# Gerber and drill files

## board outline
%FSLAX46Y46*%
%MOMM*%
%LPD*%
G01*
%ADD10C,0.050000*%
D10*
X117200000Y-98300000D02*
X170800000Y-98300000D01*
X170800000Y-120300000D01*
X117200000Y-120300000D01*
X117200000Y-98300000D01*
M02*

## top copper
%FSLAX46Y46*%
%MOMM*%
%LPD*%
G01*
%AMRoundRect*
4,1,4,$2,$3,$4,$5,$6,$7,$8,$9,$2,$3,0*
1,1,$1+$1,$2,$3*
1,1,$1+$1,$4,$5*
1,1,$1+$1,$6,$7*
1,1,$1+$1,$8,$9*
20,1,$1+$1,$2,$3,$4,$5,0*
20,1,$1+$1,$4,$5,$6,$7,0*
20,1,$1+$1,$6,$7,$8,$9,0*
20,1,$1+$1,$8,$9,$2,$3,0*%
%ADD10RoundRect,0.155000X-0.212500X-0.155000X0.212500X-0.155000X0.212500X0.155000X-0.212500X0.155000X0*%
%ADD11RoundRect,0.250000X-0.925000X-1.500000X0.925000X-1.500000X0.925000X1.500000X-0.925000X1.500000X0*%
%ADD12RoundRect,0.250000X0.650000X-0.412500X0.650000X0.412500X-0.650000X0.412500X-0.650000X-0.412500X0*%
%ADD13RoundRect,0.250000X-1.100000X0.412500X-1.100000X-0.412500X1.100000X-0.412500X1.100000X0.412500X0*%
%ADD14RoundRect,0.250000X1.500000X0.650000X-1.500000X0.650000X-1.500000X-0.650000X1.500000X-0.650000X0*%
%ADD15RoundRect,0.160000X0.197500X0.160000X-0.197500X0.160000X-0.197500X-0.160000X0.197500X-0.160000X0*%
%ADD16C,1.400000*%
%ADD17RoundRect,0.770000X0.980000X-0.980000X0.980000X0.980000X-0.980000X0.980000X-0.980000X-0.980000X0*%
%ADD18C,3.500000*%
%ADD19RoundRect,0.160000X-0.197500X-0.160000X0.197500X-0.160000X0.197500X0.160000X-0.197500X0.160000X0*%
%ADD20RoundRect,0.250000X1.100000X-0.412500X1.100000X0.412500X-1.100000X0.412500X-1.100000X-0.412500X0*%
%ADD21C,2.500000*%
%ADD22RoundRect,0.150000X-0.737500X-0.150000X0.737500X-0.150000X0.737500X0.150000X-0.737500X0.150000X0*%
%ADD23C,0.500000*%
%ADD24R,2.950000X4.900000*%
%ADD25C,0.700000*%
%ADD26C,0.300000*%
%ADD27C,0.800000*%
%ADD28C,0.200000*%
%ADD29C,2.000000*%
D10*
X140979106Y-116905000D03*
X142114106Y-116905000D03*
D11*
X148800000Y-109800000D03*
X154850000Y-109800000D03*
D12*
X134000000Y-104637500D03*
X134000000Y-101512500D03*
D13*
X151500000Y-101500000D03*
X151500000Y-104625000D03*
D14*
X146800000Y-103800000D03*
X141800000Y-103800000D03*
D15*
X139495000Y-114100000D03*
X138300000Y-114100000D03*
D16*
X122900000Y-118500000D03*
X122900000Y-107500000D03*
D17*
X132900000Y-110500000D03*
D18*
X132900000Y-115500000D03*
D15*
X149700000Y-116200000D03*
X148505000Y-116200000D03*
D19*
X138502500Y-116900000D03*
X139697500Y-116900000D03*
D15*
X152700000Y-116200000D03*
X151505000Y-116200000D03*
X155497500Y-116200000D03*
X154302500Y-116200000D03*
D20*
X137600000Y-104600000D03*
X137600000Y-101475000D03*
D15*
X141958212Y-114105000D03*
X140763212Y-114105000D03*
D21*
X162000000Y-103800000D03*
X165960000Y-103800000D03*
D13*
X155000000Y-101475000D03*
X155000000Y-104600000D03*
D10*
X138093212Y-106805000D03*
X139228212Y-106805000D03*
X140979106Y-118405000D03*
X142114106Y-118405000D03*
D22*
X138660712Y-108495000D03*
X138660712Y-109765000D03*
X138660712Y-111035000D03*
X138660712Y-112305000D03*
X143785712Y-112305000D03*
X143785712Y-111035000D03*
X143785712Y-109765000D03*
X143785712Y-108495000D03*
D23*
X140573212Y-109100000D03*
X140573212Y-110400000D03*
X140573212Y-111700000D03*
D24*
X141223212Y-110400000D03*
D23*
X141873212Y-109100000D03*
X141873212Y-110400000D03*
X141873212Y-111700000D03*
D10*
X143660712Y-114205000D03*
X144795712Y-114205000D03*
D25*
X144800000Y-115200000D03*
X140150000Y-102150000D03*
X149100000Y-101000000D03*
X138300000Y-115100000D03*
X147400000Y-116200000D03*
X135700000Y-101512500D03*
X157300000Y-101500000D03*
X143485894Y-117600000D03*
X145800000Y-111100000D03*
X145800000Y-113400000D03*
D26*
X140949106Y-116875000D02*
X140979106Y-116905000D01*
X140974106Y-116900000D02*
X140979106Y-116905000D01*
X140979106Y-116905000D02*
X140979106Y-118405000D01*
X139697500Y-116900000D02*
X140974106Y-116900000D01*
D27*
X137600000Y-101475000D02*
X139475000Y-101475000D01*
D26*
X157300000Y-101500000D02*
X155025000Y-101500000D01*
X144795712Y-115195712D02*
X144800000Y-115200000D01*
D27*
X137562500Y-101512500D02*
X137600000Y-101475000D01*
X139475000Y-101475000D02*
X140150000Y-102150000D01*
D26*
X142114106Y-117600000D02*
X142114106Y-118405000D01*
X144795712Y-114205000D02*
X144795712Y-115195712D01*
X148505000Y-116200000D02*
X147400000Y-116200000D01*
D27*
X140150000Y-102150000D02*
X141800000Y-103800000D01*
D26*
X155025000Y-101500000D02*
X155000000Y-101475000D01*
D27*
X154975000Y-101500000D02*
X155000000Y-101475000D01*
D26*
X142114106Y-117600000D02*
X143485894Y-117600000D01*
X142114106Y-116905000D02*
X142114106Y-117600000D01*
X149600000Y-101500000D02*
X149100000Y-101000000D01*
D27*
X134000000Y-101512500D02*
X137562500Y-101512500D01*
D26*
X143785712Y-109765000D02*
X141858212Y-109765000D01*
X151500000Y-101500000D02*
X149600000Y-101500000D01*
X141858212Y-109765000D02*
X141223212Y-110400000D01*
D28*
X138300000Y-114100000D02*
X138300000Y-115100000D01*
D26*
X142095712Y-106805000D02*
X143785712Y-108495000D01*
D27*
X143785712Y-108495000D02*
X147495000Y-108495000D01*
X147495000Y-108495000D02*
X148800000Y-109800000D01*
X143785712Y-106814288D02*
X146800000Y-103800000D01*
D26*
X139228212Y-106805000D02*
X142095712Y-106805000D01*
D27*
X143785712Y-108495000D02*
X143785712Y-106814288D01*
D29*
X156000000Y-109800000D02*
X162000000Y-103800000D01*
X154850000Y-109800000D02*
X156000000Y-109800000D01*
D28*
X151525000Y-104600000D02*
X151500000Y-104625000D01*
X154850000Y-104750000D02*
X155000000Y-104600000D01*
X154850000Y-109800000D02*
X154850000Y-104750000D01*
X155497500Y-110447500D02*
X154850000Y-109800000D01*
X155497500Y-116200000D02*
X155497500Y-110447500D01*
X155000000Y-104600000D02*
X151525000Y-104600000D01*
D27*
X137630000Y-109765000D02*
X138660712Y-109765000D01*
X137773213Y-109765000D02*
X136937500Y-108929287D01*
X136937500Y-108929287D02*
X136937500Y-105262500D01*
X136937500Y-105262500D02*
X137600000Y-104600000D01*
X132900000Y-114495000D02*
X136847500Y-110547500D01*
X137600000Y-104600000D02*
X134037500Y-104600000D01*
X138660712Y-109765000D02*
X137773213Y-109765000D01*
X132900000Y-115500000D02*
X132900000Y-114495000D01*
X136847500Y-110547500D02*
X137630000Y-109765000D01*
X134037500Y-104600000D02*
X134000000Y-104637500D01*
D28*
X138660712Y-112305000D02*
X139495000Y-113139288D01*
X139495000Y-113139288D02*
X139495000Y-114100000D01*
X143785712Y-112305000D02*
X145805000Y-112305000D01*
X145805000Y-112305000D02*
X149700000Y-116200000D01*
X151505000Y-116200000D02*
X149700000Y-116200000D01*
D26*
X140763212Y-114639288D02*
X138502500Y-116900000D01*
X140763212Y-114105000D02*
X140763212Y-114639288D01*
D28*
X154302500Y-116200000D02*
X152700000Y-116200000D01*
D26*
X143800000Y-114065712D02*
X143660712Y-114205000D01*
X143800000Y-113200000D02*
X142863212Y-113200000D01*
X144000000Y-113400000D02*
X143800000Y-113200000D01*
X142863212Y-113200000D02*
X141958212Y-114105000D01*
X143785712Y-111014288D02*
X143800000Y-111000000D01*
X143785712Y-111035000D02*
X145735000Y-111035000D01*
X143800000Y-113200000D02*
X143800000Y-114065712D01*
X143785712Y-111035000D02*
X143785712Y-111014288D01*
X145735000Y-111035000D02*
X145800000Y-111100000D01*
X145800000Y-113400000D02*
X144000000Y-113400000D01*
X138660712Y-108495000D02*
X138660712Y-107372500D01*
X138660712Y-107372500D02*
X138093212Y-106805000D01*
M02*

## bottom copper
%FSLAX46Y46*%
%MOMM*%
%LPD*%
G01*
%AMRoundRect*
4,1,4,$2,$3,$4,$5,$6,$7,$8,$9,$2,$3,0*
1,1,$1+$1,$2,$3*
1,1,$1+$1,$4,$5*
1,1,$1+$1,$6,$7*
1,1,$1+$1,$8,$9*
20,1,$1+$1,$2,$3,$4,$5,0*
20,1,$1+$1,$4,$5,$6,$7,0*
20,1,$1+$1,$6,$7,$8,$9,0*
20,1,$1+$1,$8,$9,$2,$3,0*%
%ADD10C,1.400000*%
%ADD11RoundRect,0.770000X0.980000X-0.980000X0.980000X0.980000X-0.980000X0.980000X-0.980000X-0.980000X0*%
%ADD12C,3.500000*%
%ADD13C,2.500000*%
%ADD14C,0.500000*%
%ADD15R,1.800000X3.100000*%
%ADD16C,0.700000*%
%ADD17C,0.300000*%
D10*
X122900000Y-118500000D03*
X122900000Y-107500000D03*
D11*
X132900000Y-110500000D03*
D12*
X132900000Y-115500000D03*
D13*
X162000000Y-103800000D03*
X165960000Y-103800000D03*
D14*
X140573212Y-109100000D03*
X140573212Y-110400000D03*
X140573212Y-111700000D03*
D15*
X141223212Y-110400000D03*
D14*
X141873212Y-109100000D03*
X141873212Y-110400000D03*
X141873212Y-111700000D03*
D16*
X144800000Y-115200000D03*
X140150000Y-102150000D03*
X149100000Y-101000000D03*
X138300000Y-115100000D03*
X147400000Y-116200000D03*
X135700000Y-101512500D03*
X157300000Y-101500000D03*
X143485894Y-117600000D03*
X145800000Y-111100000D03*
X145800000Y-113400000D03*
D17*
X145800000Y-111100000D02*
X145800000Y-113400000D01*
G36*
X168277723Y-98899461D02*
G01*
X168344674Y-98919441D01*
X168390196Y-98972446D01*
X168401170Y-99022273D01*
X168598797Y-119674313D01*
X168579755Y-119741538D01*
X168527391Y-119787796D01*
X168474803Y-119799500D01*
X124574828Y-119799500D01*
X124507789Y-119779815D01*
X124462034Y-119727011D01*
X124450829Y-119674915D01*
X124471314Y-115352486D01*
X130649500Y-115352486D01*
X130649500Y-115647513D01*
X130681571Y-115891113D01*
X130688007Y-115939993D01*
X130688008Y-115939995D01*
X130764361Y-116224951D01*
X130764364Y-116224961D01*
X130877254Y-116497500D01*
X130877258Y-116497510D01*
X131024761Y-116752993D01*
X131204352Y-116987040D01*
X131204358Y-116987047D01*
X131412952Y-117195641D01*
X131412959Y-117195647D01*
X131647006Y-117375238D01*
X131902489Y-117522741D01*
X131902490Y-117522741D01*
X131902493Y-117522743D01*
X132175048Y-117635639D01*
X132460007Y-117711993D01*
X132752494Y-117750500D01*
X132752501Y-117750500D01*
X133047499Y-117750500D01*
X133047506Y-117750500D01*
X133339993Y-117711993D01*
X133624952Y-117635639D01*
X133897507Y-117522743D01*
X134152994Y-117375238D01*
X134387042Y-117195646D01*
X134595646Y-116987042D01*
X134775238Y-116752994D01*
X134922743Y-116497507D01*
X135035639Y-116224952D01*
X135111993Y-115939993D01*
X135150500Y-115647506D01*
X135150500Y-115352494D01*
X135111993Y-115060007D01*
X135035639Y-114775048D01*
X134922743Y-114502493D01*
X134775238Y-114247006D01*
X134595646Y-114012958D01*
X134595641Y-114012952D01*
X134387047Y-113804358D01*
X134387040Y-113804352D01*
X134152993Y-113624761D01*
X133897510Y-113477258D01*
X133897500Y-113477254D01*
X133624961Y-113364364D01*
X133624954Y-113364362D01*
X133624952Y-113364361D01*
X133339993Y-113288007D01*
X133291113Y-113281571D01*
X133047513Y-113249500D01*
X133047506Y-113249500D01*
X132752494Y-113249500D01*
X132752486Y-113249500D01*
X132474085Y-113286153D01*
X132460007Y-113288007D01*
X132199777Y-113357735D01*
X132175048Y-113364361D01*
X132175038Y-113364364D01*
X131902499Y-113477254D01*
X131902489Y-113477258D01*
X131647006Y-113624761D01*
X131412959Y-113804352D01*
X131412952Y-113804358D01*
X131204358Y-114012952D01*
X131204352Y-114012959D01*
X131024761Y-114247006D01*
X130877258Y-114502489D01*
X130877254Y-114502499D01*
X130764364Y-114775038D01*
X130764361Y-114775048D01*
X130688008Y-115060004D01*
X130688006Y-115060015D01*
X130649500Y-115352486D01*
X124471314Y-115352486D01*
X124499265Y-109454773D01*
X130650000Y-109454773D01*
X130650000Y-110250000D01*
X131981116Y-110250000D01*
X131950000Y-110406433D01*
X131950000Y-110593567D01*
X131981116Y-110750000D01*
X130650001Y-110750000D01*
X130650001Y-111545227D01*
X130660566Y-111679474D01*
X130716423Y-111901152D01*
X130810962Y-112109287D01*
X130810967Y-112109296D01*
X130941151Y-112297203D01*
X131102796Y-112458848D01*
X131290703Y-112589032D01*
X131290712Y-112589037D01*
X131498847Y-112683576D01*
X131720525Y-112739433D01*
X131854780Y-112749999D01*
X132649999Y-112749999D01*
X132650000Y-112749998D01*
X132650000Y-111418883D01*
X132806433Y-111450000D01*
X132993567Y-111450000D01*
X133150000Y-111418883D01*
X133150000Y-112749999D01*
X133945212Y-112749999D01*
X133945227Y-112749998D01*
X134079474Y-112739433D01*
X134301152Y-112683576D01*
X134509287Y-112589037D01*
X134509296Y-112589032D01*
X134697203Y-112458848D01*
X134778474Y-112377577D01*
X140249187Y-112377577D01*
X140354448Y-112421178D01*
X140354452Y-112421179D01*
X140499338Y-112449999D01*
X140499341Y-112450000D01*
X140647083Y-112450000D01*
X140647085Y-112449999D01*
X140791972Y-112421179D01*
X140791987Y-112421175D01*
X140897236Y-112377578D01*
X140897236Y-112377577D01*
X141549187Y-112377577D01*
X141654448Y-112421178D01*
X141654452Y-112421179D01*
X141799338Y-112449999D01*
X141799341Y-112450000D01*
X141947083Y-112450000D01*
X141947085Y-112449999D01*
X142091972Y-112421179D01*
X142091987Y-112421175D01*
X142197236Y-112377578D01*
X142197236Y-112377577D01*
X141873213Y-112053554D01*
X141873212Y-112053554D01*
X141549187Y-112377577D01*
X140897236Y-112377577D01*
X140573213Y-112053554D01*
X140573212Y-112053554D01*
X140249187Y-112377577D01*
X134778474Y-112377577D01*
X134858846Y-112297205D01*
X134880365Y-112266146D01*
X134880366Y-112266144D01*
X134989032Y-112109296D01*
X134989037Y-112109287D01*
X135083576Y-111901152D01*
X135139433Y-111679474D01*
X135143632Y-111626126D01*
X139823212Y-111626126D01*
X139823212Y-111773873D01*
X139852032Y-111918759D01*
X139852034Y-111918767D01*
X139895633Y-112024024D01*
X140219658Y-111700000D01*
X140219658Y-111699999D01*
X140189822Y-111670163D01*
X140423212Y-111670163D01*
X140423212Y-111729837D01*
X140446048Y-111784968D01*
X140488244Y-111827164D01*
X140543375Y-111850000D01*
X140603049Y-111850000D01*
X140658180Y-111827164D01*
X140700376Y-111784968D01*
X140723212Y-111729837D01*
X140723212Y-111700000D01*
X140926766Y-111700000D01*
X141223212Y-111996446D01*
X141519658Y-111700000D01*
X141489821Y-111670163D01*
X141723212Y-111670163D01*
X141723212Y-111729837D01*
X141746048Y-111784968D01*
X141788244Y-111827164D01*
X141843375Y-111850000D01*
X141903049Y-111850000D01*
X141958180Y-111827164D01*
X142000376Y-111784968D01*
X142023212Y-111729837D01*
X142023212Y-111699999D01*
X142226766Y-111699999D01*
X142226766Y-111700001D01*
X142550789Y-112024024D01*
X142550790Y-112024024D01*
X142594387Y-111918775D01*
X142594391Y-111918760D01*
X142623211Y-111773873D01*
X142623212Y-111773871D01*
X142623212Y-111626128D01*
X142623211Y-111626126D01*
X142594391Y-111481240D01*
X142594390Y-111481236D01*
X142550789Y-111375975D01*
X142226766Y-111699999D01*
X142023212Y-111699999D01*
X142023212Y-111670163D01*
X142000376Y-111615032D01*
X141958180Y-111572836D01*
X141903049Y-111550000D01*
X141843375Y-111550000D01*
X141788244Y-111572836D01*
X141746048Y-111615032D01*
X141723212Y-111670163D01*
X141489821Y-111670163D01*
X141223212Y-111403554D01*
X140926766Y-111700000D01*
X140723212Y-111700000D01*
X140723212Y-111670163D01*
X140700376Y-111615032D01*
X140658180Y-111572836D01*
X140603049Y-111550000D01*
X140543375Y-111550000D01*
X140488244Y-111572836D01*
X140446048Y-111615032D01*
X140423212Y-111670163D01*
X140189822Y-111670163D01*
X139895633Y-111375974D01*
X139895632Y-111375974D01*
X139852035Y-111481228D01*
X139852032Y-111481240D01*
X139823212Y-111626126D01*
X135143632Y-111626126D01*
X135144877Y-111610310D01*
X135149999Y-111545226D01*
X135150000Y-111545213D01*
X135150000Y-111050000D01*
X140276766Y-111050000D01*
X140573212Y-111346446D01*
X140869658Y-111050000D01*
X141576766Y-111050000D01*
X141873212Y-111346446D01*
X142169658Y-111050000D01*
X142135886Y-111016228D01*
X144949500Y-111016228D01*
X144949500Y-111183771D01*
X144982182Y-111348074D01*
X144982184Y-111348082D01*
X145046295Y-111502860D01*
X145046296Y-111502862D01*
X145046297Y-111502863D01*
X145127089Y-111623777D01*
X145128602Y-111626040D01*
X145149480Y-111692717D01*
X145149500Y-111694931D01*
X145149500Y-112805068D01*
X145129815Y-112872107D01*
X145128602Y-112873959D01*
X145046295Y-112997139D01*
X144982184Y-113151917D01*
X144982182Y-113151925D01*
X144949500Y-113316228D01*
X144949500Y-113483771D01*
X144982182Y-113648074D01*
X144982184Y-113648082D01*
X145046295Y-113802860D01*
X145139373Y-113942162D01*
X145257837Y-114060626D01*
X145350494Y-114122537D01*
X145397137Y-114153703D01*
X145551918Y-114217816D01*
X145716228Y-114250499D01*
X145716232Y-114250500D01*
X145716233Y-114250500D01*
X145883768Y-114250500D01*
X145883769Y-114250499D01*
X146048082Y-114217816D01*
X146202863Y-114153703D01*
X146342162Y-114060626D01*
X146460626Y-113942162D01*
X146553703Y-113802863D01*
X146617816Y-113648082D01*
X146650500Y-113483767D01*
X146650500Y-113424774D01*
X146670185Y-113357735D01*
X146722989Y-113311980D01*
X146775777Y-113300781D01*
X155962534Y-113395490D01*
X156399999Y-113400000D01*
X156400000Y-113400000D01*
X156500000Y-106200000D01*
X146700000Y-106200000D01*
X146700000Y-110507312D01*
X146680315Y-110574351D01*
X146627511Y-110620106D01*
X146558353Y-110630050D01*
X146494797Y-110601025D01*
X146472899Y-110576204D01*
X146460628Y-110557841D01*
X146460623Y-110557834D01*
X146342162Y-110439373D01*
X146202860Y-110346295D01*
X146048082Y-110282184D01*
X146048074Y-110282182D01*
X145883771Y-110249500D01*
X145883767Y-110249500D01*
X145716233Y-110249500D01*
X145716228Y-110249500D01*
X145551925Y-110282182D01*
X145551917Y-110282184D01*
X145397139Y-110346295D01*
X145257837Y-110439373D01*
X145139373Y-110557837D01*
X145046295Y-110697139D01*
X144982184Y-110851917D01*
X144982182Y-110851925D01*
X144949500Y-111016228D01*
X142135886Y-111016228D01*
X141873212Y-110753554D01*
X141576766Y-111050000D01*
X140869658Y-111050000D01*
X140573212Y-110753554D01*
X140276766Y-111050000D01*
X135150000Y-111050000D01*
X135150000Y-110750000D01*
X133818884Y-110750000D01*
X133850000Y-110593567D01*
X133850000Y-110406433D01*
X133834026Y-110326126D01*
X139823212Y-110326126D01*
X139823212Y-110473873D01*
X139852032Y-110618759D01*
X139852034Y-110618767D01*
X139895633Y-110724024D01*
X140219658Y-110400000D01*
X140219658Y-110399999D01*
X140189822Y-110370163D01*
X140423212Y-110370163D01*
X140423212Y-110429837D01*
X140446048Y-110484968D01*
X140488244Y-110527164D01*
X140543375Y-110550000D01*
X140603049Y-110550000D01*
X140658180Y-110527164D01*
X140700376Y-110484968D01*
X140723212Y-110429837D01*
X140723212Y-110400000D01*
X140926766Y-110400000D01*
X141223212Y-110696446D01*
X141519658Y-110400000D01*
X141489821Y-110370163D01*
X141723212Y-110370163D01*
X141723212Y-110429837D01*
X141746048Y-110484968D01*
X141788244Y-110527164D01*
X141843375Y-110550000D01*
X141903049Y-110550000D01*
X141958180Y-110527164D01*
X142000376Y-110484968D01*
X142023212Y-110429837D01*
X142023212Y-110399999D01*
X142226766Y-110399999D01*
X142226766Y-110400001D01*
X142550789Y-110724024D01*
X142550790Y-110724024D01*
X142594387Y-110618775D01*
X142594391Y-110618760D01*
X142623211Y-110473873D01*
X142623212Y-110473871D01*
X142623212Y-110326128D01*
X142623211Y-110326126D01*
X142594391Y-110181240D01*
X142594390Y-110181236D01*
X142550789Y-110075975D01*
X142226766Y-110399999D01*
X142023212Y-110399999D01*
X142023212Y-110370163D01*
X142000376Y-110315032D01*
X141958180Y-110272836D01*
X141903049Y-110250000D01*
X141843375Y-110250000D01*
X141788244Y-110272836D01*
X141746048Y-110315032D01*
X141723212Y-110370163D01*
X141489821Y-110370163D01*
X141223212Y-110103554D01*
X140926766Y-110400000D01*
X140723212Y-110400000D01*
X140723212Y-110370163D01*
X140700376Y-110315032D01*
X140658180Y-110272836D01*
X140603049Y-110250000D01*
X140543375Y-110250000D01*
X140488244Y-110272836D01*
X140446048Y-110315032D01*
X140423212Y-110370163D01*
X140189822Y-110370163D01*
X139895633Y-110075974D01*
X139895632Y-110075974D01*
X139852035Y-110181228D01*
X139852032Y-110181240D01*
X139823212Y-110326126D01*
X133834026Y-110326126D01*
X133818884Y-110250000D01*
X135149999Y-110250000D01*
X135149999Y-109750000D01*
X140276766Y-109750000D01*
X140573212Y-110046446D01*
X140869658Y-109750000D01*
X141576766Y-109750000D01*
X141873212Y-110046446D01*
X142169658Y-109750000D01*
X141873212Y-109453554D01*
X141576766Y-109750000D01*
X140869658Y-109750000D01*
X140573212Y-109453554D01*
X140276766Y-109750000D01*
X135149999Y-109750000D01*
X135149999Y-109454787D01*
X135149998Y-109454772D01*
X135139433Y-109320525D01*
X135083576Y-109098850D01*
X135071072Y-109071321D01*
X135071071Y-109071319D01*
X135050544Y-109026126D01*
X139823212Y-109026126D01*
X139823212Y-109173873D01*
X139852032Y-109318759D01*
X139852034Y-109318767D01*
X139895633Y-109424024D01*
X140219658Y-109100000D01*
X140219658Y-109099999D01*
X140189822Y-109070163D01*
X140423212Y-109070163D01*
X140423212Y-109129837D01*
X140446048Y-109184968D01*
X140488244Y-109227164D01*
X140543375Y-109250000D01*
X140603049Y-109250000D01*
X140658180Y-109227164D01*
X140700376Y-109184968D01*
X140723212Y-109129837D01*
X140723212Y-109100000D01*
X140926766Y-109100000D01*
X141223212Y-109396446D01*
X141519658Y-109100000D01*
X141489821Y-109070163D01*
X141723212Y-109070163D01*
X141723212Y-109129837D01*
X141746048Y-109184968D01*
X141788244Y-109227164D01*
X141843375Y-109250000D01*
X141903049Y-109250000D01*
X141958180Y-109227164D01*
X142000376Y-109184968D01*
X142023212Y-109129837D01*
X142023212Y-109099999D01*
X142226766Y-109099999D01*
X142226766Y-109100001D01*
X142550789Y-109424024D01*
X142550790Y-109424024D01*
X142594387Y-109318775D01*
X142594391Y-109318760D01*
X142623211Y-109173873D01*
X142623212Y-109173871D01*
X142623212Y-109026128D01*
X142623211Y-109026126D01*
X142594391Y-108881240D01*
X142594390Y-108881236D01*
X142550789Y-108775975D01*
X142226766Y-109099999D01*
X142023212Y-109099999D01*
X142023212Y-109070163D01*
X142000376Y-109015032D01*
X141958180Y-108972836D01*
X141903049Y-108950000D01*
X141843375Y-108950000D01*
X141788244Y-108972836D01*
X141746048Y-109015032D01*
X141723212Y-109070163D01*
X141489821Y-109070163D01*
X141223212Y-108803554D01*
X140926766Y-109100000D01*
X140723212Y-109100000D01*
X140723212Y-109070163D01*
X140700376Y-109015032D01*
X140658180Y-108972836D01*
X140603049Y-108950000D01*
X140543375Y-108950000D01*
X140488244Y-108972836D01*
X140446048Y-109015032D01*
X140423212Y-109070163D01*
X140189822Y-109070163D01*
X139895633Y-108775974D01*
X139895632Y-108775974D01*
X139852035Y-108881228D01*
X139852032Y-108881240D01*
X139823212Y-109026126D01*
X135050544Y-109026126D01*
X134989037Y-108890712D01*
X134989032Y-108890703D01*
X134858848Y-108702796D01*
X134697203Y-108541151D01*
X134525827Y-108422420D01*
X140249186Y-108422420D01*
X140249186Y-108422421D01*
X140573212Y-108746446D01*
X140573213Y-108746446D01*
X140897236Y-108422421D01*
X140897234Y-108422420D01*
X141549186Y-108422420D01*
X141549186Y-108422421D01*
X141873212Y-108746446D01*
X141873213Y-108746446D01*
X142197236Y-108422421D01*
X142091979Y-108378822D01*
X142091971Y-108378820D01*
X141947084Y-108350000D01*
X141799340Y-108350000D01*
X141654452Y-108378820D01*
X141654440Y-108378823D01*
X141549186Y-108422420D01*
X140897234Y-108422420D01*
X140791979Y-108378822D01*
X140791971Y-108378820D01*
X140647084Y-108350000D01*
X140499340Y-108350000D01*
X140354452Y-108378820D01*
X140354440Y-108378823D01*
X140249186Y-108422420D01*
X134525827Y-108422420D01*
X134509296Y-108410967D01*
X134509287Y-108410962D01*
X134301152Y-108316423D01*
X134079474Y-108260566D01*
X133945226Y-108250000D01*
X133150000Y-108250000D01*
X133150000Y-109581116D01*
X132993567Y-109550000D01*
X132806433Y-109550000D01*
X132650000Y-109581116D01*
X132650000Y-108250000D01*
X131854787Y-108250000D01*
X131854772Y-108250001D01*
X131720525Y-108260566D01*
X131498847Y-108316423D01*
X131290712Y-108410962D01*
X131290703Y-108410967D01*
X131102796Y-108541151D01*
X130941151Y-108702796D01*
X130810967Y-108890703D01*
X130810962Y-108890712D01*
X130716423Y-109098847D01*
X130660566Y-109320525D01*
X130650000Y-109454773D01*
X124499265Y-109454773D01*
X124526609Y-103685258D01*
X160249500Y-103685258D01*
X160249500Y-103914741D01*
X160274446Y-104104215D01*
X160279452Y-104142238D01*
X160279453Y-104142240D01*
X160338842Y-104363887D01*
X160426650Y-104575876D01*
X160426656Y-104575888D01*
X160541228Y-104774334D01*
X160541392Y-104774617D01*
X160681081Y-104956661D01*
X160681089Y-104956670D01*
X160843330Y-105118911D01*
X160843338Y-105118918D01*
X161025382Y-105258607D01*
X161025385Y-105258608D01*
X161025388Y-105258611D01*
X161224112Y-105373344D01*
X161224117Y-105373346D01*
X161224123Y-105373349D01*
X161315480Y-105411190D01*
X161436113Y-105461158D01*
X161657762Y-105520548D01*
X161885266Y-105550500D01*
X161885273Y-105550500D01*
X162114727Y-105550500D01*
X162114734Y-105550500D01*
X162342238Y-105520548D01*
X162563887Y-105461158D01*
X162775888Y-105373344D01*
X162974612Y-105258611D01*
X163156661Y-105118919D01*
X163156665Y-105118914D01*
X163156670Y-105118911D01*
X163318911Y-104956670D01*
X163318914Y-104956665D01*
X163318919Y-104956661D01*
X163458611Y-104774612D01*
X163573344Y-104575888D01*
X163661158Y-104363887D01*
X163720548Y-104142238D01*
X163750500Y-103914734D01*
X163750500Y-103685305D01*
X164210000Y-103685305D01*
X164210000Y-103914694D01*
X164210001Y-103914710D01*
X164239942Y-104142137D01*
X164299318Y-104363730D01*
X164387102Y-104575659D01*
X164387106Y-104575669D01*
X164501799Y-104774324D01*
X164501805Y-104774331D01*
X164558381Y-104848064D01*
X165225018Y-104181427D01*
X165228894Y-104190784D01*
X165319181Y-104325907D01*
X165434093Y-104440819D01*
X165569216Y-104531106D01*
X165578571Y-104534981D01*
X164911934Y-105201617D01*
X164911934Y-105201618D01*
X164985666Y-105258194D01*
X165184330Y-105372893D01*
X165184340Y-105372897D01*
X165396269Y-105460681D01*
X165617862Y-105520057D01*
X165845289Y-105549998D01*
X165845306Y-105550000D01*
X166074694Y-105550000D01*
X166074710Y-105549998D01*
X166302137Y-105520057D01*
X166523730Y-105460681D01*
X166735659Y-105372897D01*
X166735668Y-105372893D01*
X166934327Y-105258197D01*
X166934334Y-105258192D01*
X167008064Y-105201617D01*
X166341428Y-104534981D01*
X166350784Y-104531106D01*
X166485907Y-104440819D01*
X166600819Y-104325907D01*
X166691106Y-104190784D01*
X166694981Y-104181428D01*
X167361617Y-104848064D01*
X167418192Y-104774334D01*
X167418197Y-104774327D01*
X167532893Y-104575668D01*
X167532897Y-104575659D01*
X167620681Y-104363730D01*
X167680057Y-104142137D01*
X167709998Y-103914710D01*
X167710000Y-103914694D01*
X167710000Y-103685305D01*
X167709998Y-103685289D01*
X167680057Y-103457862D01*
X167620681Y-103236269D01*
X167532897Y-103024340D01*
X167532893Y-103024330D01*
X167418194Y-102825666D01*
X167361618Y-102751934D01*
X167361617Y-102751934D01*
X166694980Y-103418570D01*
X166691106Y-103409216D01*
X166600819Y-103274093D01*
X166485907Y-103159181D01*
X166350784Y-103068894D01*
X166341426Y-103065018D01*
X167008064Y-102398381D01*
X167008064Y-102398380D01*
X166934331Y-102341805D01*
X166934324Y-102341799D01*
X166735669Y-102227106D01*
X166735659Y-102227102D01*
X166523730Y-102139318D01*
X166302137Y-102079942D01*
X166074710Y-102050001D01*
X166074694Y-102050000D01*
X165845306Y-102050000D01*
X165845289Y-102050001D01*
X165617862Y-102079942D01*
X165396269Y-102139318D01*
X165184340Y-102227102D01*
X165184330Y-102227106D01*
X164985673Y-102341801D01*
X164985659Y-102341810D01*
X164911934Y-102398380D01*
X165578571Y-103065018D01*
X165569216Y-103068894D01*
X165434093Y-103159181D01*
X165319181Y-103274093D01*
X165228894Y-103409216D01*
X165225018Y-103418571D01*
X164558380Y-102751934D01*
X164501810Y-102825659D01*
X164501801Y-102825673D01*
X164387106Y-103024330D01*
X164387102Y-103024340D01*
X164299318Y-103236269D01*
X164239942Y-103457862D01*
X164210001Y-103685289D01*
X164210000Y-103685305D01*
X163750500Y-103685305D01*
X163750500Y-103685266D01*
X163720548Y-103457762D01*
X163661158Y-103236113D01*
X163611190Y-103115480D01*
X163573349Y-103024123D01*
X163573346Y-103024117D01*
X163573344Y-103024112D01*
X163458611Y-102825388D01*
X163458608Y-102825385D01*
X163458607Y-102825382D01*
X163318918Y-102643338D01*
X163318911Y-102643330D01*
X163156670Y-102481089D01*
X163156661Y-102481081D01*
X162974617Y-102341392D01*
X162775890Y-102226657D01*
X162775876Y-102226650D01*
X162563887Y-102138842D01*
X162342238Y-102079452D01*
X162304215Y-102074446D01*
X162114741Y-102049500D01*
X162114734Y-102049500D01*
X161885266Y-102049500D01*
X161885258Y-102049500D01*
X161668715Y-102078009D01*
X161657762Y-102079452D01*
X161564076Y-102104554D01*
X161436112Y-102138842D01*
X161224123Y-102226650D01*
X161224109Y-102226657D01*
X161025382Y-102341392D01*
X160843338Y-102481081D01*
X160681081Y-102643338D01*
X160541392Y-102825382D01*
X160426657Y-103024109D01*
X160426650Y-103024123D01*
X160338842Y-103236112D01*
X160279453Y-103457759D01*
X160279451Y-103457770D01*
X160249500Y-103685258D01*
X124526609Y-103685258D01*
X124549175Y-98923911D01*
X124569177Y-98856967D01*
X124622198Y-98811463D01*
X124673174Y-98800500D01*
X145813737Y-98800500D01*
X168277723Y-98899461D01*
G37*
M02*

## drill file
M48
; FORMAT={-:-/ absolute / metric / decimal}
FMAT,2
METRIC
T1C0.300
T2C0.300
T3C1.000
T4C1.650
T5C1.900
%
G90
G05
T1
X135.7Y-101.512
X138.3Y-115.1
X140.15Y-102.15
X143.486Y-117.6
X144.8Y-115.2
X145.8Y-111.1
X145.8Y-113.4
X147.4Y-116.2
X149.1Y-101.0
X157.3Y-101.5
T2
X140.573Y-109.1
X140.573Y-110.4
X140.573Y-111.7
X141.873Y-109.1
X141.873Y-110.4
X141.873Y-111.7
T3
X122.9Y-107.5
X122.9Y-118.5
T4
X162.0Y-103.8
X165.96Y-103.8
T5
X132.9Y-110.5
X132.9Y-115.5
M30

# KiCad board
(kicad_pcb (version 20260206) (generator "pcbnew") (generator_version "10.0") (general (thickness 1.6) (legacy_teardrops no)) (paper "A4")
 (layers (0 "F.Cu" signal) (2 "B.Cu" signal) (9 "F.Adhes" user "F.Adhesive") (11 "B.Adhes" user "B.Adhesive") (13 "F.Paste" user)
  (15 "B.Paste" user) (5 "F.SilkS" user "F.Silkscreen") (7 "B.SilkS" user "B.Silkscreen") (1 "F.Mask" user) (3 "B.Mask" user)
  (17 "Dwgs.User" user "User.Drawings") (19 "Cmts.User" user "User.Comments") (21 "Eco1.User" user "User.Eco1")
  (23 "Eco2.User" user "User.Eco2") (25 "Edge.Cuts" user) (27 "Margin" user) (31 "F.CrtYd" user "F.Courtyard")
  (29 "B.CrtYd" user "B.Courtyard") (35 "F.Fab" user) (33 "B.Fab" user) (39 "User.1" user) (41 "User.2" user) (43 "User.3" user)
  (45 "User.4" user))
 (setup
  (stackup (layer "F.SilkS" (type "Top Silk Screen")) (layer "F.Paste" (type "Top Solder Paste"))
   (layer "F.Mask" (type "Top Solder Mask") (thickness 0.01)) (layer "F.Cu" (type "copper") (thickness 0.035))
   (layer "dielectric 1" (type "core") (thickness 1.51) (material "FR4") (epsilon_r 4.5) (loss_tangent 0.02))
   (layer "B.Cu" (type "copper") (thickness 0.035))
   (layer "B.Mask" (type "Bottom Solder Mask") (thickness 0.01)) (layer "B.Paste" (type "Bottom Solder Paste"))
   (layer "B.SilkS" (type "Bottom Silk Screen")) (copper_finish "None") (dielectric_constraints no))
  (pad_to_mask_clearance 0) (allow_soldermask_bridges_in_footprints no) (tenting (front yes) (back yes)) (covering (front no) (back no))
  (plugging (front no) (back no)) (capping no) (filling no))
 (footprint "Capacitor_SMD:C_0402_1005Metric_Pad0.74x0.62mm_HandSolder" (layer "F.Cu") (at 141.546606 116.905)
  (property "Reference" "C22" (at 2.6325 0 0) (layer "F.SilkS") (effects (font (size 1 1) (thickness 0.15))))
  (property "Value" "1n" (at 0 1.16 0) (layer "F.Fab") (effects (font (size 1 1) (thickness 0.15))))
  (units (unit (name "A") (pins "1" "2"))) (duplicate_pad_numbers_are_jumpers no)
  (pad "1" smd roundrect (at -0.5675 0) (size 0.735 0.62) (layers "F.Cu" "F.Mask" "F.Paste") (roundrect_rratio 0.25) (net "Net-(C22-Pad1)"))
  (pad "2" smd roundrect (at 0.5675 0) (size 0.735 0.62) (layers "F.Cu" "F.Mask" "F.Paste") (roundrect_rratio 0.25) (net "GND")))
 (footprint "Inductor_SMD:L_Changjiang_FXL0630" (layer "F.Cu") (at 151.825 109.8)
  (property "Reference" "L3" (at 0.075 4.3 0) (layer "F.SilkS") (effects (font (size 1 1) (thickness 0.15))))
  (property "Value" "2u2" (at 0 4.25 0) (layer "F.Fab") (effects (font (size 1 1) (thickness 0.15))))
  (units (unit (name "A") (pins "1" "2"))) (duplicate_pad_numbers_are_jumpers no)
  (pad "1" smd roundrect (at -3.025 0) (size 2.35 3.5) (layers "F.Cu" "F.Mask" "F.Paste") (roundrect_rratio 0.106383) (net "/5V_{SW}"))
  (pad "2" smd roundrect (at 3.025 0) (size 2.35 3.5) (layers "F.Cu" "F.Mask" "F.Paste") (roundrect_rratio 0.106383) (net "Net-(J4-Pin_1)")))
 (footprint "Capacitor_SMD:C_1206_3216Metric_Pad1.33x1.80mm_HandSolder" (layer "F.Cu") (at 134 103.075 90)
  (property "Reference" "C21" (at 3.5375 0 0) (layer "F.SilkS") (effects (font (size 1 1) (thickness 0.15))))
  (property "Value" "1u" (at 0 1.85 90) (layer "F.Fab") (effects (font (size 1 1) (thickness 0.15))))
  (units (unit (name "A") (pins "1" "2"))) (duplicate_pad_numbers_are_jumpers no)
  (pad "1" smd roundrect (at -1.5625 0 90) (size 1.325 1.8) (layers "F.Cu" "F.Mask" "F.Paste") (roundrect_rratio 0.188679) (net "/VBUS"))
  (pad "2" smd roundrect (at 1.5625 0 90) (size 1.325 1.8) (layers "F.Cu" "F.Mask" "F.Paste") (roundrect_rratio 0.188679) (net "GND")))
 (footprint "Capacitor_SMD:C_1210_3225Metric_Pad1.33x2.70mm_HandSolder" (layer "F.Cu") (at 151.5 103.0625 -90)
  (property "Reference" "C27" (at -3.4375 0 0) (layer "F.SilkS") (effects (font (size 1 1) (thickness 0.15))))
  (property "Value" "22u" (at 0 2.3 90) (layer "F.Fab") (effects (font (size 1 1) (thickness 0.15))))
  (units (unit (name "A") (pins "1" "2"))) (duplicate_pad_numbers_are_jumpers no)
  (pad "1" smd roundrect (at -1.5625 0 270) (size 1.325 2.7) (layers "F.Cu" "F.Mask" "F.Paste") (roundrect_rratio 0.188679) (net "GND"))
  (pad "2" smd roundrect (at 1.5625 0 270) (size 1.325 2.7) (layers "F.Cu" "F.Mask" "F.Paste") (roundrect_rratio 0.188679)
   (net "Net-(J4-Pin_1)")))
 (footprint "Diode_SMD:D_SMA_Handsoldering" (layer "F.Cu") (at 144.3 103.8 180)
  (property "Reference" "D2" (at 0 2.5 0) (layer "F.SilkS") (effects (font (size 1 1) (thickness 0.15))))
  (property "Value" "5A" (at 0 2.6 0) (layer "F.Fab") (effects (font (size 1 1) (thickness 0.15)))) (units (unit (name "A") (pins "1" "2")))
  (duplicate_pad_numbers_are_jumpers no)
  (pad "1" smd roundrect (at -2.5 0 180) (size 3.5 1.8) (layers "F.Cu" "F.Mask" "F.Paste") (roundrect_rratio 0.1388888889) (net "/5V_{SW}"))
  (pad "2" smd roundrect (at 2.5 0 180) (size 3.5 1.8) (layers "F.Cu" "F.Mask" "F.Paste") (roundrect_rratio 0.1388888889) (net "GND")))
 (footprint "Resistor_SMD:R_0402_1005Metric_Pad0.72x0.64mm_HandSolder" (layer "F.Cu") (at 138.8975 114.1 180)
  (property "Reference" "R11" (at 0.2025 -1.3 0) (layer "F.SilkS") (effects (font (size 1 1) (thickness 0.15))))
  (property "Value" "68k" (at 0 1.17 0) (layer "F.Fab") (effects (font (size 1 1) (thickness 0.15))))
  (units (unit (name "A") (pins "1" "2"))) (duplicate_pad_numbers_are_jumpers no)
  (pad "1" smd roundrect (at -0.5975 0 180) (size 0.715 0.64) (layers "F.Cu" "F.Mask" "F.Paste") (roundrect_rratio 0.25) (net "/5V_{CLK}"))
  (pad "2" smd roundrect (at 0.5975 0 180) (size 0.715 0.64) (layers "F.Cu" "F.Mask" "F.Paste") (roundrect_rratio 0.25) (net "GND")))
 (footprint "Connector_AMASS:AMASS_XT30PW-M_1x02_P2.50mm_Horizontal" (layer "F.Cu") (at 132.9 110.5 90)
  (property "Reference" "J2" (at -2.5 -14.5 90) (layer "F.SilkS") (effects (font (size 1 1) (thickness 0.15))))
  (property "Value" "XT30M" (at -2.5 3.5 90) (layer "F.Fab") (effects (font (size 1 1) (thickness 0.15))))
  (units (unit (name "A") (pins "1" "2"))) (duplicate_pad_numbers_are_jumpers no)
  (pad "" thru_hole circle (at -8 -10 90) (size 1.4 1.4) (drill 1) (layers "*.Cu" "*.Mask") (remove_unused_layers no))
  (pad "" thru_hole circle (at 3 -10 90) (size 1.4 1.4) (drill 1) (layers "*.Cu" "*.Mask") (remove_unused_layers no))
  (pad "1" thru_hole roundrect (at 0 0 90) (size 3.5 3.5) (drill 1.9) (layers "*.Cu" "*.Mask") (remove_unused_layers no)
   (roundrect_rratio 0.22) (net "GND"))
  (pad "2" thru_hole circle (at -5 0 90) (size 3.5 3.5) (drill 1.9) (layers "*.Cu" "*.Mask") (remove_unused_layers no) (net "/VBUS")))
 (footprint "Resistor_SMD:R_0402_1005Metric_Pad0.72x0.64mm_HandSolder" (layer "F.Cu") (at 149.1025 116.2 180)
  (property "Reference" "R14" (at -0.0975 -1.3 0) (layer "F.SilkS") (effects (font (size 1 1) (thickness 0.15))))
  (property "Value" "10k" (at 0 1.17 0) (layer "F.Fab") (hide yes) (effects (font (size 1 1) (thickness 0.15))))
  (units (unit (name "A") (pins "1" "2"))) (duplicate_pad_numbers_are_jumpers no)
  (pad "1" smd roundrect (at -0.5975 0 180) (size 0.715 0.64) (layers "F.Cu" "F.Mask" "F.Paste") (roundrect_rratio 0.25) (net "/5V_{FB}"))
  (pad "2" smd roundrect (at 0.5975 0 180) (size 0.715 0.64) (layers "F.Cu" "F.Mask" "F.Paste") (roundrect_rratio 0.25) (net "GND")))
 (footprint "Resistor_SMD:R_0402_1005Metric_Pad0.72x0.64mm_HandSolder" (layer "F.Cu") (at 139.1 116.9)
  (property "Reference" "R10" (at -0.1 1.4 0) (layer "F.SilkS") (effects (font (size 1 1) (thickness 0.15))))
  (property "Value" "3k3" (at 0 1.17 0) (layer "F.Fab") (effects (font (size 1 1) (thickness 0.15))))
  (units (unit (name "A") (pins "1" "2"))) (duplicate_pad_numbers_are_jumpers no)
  (pad "1" smd roundrect (at -0.5975 0) (size 0.715 0.64) (layers "F.Cu" "F.Mask" "F.Paste") (roundrect_rratio 0.25) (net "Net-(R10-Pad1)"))
  (pad "2" smd roundrect (at 0.5975 0) (size 0.715 0.64) (layers "F.Cu" "F.Mask" "F.Paste") (roundrect_rratio 0.25) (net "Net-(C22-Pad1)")))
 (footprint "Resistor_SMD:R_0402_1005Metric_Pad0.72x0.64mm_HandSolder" (layer "F.Cu") (at 152.1025 116.2 180)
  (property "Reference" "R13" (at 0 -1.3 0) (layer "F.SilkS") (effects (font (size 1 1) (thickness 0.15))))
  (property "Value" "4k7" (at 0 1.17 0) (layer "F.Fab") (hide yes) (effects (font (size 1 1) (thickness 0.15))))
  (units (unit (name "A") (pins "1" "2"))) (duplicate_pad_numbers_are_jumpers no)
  (pad "1" smd roundrect (at -0.5975 0 180) (size 0.715 0.64) (layers "F.Cu" "F.Mask" "F.Paste") (roundrect_rratio 0.25)
   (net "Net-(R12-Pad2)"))
  (pad "2" smd roundrect (at 0.5975 0 180) (size 0.715 0.64) (layers "F.Cu" "F.Mask" "F.Paste") (roundrect_rratio 0.25) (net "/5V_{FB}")))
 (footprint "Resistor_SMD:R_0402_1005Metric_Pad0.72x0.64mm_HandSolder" (layer "F.Cu") (at 154.9 116.2 180)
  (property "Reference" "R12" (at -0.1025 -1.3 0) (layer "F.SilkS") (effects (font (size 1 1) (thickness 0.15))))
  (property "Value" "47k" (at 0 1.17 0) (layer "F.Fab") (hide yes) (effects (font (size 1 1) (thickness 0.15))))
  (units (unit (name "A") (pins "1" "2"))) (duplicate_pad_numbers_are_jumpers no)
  (pad "1" smd roundrect (at -0.5975 0 180) (size 0.715 0.64) (layers "F.Cu" "F.Mask" "F.Paste") (roundrect_rratio 0.25)
   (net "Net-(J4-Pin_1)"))
  (pad "2" smd roundrect (at 0.5975 0 180) (size 0.715 0.64) (layers "F.Cu" "F.Mask" "F.Paste") (roundrect_rratio 0.25)
   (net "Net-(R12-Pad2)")))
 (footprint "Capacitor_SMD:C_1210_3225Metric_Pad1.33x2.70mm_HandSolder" (layer "F.Cu") (at 137.6 103.0375 90)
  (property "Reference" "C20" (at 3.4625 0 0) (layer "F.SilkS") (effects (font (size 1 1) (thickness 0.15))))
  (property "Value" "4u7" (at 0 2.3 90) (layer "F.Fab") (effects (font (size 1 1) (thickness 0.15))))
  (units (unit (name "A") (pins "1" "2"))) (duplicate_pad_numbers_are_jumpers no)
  (pad "1" smd roundrect (at -1.5625 0 90) (size 1.325 2.7) (layers "F.Cu" "F.Mask" "F.Paste") (roundrect_rratio 0.188679) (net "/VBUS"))
  (pad "2" smd roundrect (at 1.5625 0 90) (size 1.325 2.7) (layers "F.Cu" "F.Mask" "F.Paste") (roundrect_rratio 0.188679) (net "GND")))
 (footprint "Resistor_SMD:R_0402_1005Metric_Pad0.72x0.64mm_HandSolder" (layer "F.Cu") (at 141.360712 114.105 180)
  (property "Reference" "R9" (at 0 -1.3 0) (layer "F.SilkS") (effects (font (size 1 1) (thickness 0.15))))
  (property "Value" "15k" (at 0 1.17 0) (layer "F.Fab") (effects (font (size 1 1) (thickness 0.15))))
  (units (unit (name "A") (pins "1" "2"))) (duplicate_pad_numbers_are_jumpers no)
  (pad "1" smd roundrect (at -0.5975 0 180) (size 0.715 0.64) (layers "F.Cu" "F.Mask" "F.Paste") (roundrect_rratio 0.25) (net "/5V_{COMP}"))
  (pad "2" smd roundrect (at 0.5975 0 180) (size 0.715 0.64) (layers "F.Cu" "F.Mask" "F.Paste") (roundrect_rratio 0.25)
   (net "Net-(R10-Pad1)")))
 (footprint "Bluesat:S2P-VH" (layer "F.Cu") (at 163.98 117.3 180)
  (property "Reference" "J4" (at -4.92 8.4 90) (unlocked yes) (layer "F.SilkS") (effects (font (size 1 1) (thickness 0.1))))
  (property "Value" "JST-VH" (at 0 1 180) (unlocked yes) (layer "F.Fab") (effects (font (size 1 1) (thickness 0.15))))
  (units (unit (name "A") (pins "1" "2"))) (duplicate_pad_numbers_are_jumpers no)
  (pad "1" thru_hole circle (at 1.98 13.5 180) (size 2.5 2.5) (drill 1.65) (layers "*.Cu" "*.Mask") (remove_unused_layers no)
   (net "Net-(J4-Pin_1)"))
  (pad "2" thru_hole circle (at -1.98 13.5 180) (size 2.5 2.5) (drill 1.65) (layers "*.Cu" "*.Mask") (remove_unused_layers no) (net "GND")))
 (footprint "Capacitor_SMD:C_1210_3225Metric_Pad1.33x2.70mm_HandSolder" (layer "F.Cu") (at 155 103.0375 -90)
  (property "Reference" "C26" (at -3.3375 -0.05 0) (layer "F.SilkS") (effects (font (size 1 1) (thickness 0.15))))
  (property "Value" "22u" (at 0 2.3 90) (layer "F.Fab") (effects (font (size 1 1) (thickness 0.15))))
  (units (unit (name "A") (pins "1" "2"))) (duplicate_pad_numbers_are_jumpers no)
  (pad "1" smd roundrect (at -1.5625 0 270) (size 1.325 2.7) (layers "F.Cu" "F.Mask" "F.Paste") (roundrect_rratio 0.188679) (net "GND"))
  (pad "2" smd roundrect (at 1.5625 0 270) (size 1.325 2.7) (layers "F.Cu" "F.Mask" "F.Paste") (roundrect_rratio 0.188679)
   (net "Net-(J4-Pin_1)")))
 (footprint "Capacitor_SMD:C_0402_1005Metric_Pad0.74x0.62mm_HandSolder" (layer "F.Cu") (at 138.660712 106.805)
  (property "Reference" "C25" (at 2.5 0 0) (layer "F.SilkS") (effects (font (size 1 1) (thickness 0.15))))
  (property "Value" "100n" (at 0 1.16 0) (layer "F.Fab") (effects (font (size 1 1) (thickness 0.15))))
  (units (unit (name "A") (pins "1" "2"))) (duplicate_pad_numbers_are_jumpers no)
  (pad "1" smd roundrect (at -0.5675 0) (size 0.735 0.62) (layers "F.Cu" "F.Mask" "F.Paste") (roundrect_rratio 0.25) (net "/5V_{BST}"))
  (pad "2" smd roundrect (at 0.5675 0) (size 0.735 0.62) (layers "F.Cu" "F.Mask" "F.Paste") (roundrect_rratio 0.25) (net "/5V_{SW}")))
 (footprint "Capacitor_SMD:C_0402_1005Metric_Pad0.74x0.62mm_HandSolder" (layer "F.Cu") (at 141.546606 118.405)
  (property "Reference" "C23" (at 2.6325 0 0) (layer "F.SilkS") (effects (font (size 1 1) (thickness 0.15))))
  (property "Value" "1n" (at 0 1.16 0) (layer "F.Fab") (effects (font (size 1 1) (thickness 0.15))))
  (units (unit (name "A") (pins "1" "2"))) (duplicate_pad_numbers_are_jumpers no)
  (pad "1" smd roundrect (at -0.5675 0) (size 0.735 0.62) (layers "F.Cu" "F.Mask" "F.Paste") (roundrect_rratio 0.25) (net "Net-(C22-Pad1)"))
  (pad "2" smd roundrect (at 0.5675 0) (size 0.735 0.62) (layers "F.Cu" "F.Mask" "F.Paste") (roundrect_rratio 0.25) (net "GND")))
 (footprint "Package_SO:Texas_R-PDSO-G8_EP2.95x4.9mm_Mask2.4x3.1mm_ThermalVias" (layer "F.Cu") (at 141.223212 110.4)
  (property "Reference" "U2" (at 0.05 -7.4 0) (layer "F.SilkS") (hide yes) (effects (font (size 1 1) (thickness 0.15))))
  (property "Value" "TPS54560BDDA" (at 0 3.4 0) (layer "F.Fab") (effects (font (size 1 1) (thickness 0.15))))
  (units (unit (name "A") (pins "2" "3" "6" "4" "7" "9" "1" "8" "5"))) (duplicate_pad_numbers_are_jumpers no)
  (pad "" smd roundrect (at -0.6 -1.03) (size 1.04 0.89) (layers "F.Paste") (roundrect_rratio 0.25))
  (pad "" smd roundrect (at -0.6 0) (size 1.04 0.89) (layers "F.Paste") (roundrect_rratio 0.25))
  (pad "" smd roundrect (at -0.6 1.03) (size 1.04 0.89) (layers "F.Paste") (roundrect_rratio 0.25))
  (pad "" smd rect (at 0 0) (size 2.4 3.1) (layers "F.Mask"))
  (pad "" smd roundrect (at 0.6 -1.03) (size 1.04 0.89) (layers "F.Paste") (roundrect_rratio 0.25))
  (pad "" smd roundrect (at 0.6 0) (size 1.04 0.89) (layers "F.Paste") (roundrect_rratio 0.25))
  (pad "" smd roundrect (at 0.6 1.03) (size 1.04 0.89) (layers "F.Paste") (roundrect_rratio 0.25))
  (pad "1" smd roundrect (at -2.5625 -1.905) (size 1.775 0.6) (layers "F.Cu" "F.Mask" "F.Paste") (roundrect_rratio 0.25) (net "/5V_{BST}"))
  (pad "2" smd roundrect (at -2.5625 -0.635) (size 1.775 0.6) (layers "F.Cu" "F.Mask" "F.Paste") (roundrect_rratio 0.25) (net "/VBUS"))
  (pad "3" smd roundrect (at -2.5625 0.635) (size 1.775 0.6) (layers "F.Cu" "F.Mask" "F.Paste") (roundrect_rratio 0.25)
   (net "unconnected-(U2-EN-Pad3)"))
  (pad "4" smd roundrect (at -2.5625 1.905) (size 1.775 0.6) (layers "F.Cu" "F.Mask" "F.Paste") (roundrect_rratio 0.25) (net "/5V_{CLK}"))
  (pad "5" smd roundrect (at 2.5625 1.905) (size 1.775 0.6) (layers "F.Cu" "F.Mask" "F.Paste") (roundrect_rratio 0.25) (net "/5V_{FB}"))
  (pad "6" smd roundrect (at 2.5625 0.635) (size 1.775 0.6) (layers "F.Cu" "F.Mask" "F.Paste") (roundrect_rratio 0.25) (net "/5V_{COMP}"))
  (pad "7" smd roundrect (at 2.5625 -0.635) (size 1.775 0.6) (layers "F.Cu" "F.Mask" "F.Paste") (roundrect_rratio 0.25) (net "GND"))
  (pad "8" smd roundrect (at 2.5625 -1.905) (size 1.775 0.6) (layers "F.Cu" "F.Mask" "F.Paste") (roundrect_rratio 0.25) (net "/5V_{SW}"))
  (pad "9" thru_hole circle (at -0.65 -1.3) (size 0.5 0.5) (drill 0.3) (layers "*.Cu") (remove_unused_layers no) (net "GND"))
  (pad "9" thru_hole circle (at -0.65 0) (size 0.5 0.5) (drill 0.3) (layers "*.Cu") (remove_unused_layers no) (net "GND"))
  (pad "9" thru_hole circle (at -0.65 1.3) (size 0.5 0.5) (drill 0.3) (layers "*.Cu") (remove_unused_layers no) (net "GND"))
  (pad "9" smd rect (at 0 0) (size 1.8 3.1) (layers "B.Cu") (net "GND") (zone_connect 2))
  (pad "9" smd rect (at 0 0) (size 2.95 4.9) (layers "F.Cu") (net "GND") (zone_connect 2))
  (pad "9" thru_hole circle (at 0.65 -1.3) (size 0.5 0.5) (drill 0.3) (layers "*.Cu") (remove_unused_layers no) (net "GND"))
  (pad "9" thru_hole circle (at 0.65 0) (size 0.5 0.5) (drill 0.3) (layers "*.Cu") (remove_unused_layers no) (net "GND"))
  (pad "9" thru_hole circle (at 0.65 1.3) (size 0.5 0.5) (drill 0.3) (layers "*.Cu") (remove_unused_layers no) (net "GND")))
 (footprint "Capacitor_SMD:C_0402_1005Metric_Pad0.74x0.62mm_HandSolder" (layer "F.Cu") (at 144.228212 114.205)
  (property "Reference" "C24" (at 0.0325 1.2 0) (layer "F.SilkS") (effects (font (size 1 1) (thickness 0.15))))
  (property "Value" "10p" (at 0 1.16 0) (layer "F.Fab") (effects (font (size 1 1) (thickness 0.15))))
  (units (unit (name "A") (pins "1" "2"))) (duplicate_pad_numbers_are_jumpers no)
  (pad "1" smd roundrect (at -0.5675 0) (size 0.735 0.62) (layers "F.Cu" "F.Mask" "F.Paste") (roundrect_rratio 0.25) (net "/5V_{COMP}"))
  (pad "2" smd roundrect (at 0.5675 0) (size 0.735 0.62) (layers "F.Cu" "F.Mask" "F.Paste") (roundrect_rratio 0.25) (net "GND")))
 (gr_rect (start 117.2 98.3) (end 170.8 120.3) (stroke (width 0.05) (type default)) (fill no) (layer "Edge.Cuts"))
 (segment (start 140.949106 116.875) (end 140.979106 116.905) (width 0.3) (layer "F.Cu") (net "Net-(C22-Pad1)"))
 (segment (start 140.974106 116.9) (end 140.979106 116.905) (width 0.3) (layer "F.Cu") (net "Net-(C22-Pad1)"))
 (segment (start 140.979106 116.905) (end 140.979106 118.405) (width 0.3) (layer "F.Cu") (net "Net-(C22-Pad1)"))
 (segment (start 139.6975 116.9) (end 140.974106 116.9) (width 0.3) (layer "F.Cu") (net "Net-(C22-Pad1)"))
 (segment (start 137.6 101.475) (end 139.475 101.475) (width 0.8) (layer "F.Cu") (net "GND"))
 (segment (start 157.3 101.5) (end 155.025 101.5) (width 0.3) (layer "F.Cu") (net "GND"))
 (segment (start 144.795712 115.195712) (end 144.8 115.2) (width 0.3) (layer "F.Cu") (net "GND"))
 (segment (start 137.5625 101.5125) (end 137.6 101.475) (width 0.8) (layer "F.Cu") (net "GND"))
 (segment (start 139.475 101.475) (end 140.15 102.15) (width 0.8) (layer "F.Cu") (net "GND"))
 (segment (start 142.114106 117.6) (end 142.114106 118.405) (width 0.3) (layer "F.Cu") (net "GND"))
 (segment (start 144.795712 114.205) (end 144.795712 115.195712) (width 0.3) (layer "F.Cu") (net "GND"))
 (segment (start 148.505 116.2) (end 147.4 116.2) (width 0.3) (layer "F.Cu") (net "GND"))
 (segment (start 140.15 102.15) (end 141.8 103.8) (width 0.8) (layer "F.Cu") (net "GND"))
 (segment (start 155.025 101.5) (end 155 101.475) (width 0.3) (layer "F.Cu") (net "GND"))
 (segment (start 154.975 101.5) (end 155 101.475) (width 0.8) (layer "F.Cu") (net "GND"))
 (segment (start 142.114106 117.6) (end 143.485894 117.6) (width 0.3) (layer "F.Cu") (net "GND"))
 (segment (start 142.114106 116.905) (end 142.114106 117.6) (width 0.3) (layer "F.Cu") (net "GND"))
 (segment (start 149.6 101.5) (end 149.1 101) (width 0.3) (layer "F.Cu") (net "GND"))
 (segment (start 134 101.5125) (end 137.5625 101.5125) (width 0.8) (layer "F.Cu") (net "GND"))
 (segment (start 143.785712 109.765) (end 141.858212 109.765) (width 0.3) (layer "F.Cu") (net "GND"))
 (segment (start 151.5 101.5) (end 149.6 101.5) (width 0.3) (layer "F.Cu") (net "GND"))
 (segment (start 141.858212 109.765) (end 141.223212 110.4) (width 0.3) (layer "F.Cu") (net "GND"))
 (segment (start 138.3 114.1) (end 138.3 115.1) (width 0.2) (layer "F.Cu") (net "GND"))
 (via (at 144.8 115.2) (size 0.7) (drill 0.3) (layers "F.Cu" "B.Cu") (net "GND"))
 (via (at 140.15 102.15) (size 0.7) (drill 0.3) (layers "F.Cu" "B.Cu") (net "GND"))
 (via (at 149.1 101) (size 0.7) (drill 0.3) (layers "F.Cu" "B.Cu") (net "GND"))
 (via (at 138.3 115.1) (size 0.7) (drill 0.3) (layers "F.Cu" "B.Cu") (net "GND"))
 (via (at 147.4 116.2) (size 0.7) (drill 0.3) (layers "F.Cu" "B.Cu") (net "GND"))
 (via (at 135.7 101.5125) (size 0.7) (drill 0.3) (layers "F.Cu" "B.Cu") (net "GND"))
 (via (at 157.3 101.5) (size 0.7) (drill 0.3) (layers "F.Cu" "B.Cu") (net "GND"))
 (via (at 143.485894 117.6) (size 0.7) (drill 0.3) (layers "F.Cu" "B.Cu") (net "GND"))
 (segment (start 142.095712 106.805) (end 143.785712 108.495) (width 0.3) (layer "F.Cu") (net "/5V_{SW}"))
 (segment (start 143.785712 108.495) (end 147.495 108.495) (width 0.8) (layer "F.Cu") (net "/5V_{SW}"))
 (segment (start 147.495 108.495) (end 148.8 109.8) (width 0.8) (layer "F.Cu") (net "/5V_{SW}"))
 (segment (start 143.785712 106.814288) (end 146.8 103.8) (width 0.8) (layer "F.Cu") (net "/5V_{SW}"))
 (segment (start 139.228212 106.805) (end 142.095712 106.805) (width 0.3) (layer "F.Cu") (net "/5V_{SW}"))
 (segment (start 143.785712 108.495) (end 143.785712 106.814288) (width 0.8) (layer "F.Cu") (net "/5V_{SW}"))
 (segment (start 156 109.8) (end 162 103.8) (width 2) (layer "F.Cu") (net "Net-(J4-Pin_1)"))
 (segment (start 154.85 109.8) (end 156 109.8) (width 2) (layer "F.Cu") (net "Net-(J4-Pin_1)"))
 (segment (start 151.525 104.6) (end 151.5 104.625) (width 0.2) (layer "F.Cu") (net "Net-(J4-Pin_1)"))
 (segment (start 154.85 104.75) (end 155 104.6) (width 0.2) (layer "F.Cu") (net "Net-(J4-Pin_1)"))
 (segment (start 154.85 109.8) (end 154.85 104.75) (width 0.2) (layer "F.Cu") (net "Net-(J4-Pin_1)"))
 (segment (start 155.4975 110.4475) (end 154.85 109.8) (width 0.2) (layer "F.Cu") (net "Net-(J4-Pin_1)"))
 (segment (start 155.4975 116.2) (end 155.4975 110.4475) (width 0.2) (layer "F.Cu") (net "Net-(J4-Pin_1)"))
 (segment (start 155 104.6) (end 151.525 104.6) (width 0.2) (layer "F.Cu") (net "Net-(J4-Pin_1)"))
 (segment (start 137.63 109.765) (end 138.660712 109.765) (width 0.8) (layer "F.Cu") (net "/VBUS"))
 (segment (start 137.773213 109.765) (end 136.9375 108.929287) (width 0.8) (layer "F.Cu") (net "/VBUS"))
 (segment (start 136.9375 108.929287) (end 136.9375 105.2625) (width 0.8) (layer "F.Cu") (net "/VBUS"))
 (segment (start 136.9375 105.2625) (end 137.6 104.6) (width 0.8) (layer "F.Cu") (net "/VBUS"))
 (segment (start 132.9 114.495) (end 136.8475 110.5475) (width 0.8) (layer "F.Cu") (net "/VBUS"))
 (segment (start 137.6 104.6) (end 134.0375 104.6) (width 0.8) (layer "F.Cu") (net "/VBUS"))
 (segment (start 138.660712 109.765) (end 137.773213 109.765) (width 0.8) (layer "F.Cu") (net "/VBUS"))
 (segment (start 132.9 115.5) (end 132.9 114.495) (width 0.8) (layer "F.Cu") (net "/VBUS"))
 (segment (start 136.8475 110.5475) (end 137.63 109.765) (width 0.8) (layer "F.Cu") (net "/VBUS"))
 (segment (start 134.0375 104.6) (end 134 104.6375) (width 0.8) (layer "F.Cu") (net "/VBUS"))
 (segment (start 138.660712 112.305) (end 139.495 113.139288) (width 0.2) (layer "F.Cu") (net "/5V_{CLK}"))
 (segment (start 139.495 113.139288) (end 139.495 114.1) (width 0.2) (layer "F.Cu") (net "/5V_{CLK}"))
 (segment (start 143.785712 112.305) (end 145.805 112.305) (width 0.2) (layer "F.Cu") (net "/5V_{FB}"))
 (segment (start 145.805 112.305) (end 149.7 116.2) (width 0.2) (layer "F.Cu") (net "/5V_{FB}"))
 (segment (start 151.505 116.2) (end 149.7 116.2) (width 0.2) (layer "F.Cu") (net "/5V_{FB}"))
 (segment (start 140.763212 114.639288) (end 138.5025 116.9) (width 0.3) (layer "F.Cu") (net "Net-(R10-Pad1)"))
 (segment (start 140.763212 114.105) (end 140.763212 114.639288) (width 0.3) (layer "F.Cu") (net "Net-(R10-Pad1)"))
 (segment (start 154.3025 116.2) (end 152.7 116.2) (width 0.2) (layer "F.Cu") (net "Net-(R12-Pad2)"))
 (segment (start 143.8 114.065712) (end 143.660712 114.205) (width 0.3) (layer "F.Cu") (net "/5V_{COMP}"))
 (segment (start 143.8 113.2) (end 142.863212 113.2) (width 0.3) (layer "F.Cu") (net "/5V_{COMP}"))
 (segment (start 144 113.4) (end 143.8 113.2) (width 0.3) (layer "F.Cu") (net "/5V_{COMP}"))
 (segment (start 142.863212 113.2) (end 141.958212 114.105) (width 0.3) (layer "F.Cu") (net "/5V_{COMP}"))
 (segment (start 143.785712 111.014288) (end 143.8 111) (width 0.3) (layer "F.Cu") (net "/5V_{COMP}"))
 (segment (start 143.785712 111.035) (end 145.735 111.035) (width 0.3) (layer "F.Cu") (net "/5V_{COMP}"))
 (segment (start 143.8 113.2) (end 143.8 114.065712) (width 0.3) (layer "F.Cu") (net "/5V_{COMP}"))
 (segment (start 143.785712 111.035) (end 143.785712 111.014288) (width 0.3) (layer "F.Cu") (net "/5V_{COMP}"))
 (segment (start 145.735 111.035) (end 145.8 111.1) (width 0.3) (layer "F.Cu") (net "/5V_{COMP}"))
 (segment (start 145.8 113.4) (end 144 113.4) (width 0.3) (layer "F.Cu") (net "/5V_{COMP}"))
 (via (at 145.8 111.1) (size 0.7) (drill 0.3) (layers "F.Cu" "B.Cu") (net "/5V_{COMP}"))
 (via (at 145.8 113.4) (size 0.7) (drill 0.3) (layers "F.Cu" "B.Cu") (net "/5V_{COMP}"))
 (segment (start 145.8 111.1) (end 145.8 113.4) (width 0.3) (layer "B.Cu") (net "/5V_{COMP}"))
 (segment (start 138.660712 108.495) (end 138.660712 107.3725) (width 0.3) (layer "F.Cu") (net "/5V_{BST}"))
 (segment (start 138.660712 107.3725) (end 138.093212 106.805) (width 0.3) (layer "F.Cu") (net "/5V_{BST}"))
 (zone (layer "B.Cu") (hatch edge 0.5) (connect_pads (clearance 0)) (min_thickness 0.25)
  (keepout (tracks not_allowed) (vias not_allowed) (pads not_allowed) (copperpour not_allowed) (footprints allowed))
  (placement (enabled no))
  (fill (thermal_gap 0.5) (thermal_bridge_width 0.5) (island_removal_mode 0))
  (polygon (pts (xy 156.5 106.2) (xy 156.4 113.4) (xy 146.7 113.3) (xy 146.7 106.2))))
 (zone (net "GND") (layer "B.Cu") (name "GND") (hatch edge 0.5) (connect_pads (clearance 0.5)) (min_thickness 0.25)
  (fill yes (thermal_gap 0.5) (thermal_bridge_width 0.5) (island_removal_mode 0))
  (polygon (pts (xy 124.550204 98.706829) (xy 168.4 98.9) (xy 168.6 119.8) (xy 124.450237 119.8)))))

